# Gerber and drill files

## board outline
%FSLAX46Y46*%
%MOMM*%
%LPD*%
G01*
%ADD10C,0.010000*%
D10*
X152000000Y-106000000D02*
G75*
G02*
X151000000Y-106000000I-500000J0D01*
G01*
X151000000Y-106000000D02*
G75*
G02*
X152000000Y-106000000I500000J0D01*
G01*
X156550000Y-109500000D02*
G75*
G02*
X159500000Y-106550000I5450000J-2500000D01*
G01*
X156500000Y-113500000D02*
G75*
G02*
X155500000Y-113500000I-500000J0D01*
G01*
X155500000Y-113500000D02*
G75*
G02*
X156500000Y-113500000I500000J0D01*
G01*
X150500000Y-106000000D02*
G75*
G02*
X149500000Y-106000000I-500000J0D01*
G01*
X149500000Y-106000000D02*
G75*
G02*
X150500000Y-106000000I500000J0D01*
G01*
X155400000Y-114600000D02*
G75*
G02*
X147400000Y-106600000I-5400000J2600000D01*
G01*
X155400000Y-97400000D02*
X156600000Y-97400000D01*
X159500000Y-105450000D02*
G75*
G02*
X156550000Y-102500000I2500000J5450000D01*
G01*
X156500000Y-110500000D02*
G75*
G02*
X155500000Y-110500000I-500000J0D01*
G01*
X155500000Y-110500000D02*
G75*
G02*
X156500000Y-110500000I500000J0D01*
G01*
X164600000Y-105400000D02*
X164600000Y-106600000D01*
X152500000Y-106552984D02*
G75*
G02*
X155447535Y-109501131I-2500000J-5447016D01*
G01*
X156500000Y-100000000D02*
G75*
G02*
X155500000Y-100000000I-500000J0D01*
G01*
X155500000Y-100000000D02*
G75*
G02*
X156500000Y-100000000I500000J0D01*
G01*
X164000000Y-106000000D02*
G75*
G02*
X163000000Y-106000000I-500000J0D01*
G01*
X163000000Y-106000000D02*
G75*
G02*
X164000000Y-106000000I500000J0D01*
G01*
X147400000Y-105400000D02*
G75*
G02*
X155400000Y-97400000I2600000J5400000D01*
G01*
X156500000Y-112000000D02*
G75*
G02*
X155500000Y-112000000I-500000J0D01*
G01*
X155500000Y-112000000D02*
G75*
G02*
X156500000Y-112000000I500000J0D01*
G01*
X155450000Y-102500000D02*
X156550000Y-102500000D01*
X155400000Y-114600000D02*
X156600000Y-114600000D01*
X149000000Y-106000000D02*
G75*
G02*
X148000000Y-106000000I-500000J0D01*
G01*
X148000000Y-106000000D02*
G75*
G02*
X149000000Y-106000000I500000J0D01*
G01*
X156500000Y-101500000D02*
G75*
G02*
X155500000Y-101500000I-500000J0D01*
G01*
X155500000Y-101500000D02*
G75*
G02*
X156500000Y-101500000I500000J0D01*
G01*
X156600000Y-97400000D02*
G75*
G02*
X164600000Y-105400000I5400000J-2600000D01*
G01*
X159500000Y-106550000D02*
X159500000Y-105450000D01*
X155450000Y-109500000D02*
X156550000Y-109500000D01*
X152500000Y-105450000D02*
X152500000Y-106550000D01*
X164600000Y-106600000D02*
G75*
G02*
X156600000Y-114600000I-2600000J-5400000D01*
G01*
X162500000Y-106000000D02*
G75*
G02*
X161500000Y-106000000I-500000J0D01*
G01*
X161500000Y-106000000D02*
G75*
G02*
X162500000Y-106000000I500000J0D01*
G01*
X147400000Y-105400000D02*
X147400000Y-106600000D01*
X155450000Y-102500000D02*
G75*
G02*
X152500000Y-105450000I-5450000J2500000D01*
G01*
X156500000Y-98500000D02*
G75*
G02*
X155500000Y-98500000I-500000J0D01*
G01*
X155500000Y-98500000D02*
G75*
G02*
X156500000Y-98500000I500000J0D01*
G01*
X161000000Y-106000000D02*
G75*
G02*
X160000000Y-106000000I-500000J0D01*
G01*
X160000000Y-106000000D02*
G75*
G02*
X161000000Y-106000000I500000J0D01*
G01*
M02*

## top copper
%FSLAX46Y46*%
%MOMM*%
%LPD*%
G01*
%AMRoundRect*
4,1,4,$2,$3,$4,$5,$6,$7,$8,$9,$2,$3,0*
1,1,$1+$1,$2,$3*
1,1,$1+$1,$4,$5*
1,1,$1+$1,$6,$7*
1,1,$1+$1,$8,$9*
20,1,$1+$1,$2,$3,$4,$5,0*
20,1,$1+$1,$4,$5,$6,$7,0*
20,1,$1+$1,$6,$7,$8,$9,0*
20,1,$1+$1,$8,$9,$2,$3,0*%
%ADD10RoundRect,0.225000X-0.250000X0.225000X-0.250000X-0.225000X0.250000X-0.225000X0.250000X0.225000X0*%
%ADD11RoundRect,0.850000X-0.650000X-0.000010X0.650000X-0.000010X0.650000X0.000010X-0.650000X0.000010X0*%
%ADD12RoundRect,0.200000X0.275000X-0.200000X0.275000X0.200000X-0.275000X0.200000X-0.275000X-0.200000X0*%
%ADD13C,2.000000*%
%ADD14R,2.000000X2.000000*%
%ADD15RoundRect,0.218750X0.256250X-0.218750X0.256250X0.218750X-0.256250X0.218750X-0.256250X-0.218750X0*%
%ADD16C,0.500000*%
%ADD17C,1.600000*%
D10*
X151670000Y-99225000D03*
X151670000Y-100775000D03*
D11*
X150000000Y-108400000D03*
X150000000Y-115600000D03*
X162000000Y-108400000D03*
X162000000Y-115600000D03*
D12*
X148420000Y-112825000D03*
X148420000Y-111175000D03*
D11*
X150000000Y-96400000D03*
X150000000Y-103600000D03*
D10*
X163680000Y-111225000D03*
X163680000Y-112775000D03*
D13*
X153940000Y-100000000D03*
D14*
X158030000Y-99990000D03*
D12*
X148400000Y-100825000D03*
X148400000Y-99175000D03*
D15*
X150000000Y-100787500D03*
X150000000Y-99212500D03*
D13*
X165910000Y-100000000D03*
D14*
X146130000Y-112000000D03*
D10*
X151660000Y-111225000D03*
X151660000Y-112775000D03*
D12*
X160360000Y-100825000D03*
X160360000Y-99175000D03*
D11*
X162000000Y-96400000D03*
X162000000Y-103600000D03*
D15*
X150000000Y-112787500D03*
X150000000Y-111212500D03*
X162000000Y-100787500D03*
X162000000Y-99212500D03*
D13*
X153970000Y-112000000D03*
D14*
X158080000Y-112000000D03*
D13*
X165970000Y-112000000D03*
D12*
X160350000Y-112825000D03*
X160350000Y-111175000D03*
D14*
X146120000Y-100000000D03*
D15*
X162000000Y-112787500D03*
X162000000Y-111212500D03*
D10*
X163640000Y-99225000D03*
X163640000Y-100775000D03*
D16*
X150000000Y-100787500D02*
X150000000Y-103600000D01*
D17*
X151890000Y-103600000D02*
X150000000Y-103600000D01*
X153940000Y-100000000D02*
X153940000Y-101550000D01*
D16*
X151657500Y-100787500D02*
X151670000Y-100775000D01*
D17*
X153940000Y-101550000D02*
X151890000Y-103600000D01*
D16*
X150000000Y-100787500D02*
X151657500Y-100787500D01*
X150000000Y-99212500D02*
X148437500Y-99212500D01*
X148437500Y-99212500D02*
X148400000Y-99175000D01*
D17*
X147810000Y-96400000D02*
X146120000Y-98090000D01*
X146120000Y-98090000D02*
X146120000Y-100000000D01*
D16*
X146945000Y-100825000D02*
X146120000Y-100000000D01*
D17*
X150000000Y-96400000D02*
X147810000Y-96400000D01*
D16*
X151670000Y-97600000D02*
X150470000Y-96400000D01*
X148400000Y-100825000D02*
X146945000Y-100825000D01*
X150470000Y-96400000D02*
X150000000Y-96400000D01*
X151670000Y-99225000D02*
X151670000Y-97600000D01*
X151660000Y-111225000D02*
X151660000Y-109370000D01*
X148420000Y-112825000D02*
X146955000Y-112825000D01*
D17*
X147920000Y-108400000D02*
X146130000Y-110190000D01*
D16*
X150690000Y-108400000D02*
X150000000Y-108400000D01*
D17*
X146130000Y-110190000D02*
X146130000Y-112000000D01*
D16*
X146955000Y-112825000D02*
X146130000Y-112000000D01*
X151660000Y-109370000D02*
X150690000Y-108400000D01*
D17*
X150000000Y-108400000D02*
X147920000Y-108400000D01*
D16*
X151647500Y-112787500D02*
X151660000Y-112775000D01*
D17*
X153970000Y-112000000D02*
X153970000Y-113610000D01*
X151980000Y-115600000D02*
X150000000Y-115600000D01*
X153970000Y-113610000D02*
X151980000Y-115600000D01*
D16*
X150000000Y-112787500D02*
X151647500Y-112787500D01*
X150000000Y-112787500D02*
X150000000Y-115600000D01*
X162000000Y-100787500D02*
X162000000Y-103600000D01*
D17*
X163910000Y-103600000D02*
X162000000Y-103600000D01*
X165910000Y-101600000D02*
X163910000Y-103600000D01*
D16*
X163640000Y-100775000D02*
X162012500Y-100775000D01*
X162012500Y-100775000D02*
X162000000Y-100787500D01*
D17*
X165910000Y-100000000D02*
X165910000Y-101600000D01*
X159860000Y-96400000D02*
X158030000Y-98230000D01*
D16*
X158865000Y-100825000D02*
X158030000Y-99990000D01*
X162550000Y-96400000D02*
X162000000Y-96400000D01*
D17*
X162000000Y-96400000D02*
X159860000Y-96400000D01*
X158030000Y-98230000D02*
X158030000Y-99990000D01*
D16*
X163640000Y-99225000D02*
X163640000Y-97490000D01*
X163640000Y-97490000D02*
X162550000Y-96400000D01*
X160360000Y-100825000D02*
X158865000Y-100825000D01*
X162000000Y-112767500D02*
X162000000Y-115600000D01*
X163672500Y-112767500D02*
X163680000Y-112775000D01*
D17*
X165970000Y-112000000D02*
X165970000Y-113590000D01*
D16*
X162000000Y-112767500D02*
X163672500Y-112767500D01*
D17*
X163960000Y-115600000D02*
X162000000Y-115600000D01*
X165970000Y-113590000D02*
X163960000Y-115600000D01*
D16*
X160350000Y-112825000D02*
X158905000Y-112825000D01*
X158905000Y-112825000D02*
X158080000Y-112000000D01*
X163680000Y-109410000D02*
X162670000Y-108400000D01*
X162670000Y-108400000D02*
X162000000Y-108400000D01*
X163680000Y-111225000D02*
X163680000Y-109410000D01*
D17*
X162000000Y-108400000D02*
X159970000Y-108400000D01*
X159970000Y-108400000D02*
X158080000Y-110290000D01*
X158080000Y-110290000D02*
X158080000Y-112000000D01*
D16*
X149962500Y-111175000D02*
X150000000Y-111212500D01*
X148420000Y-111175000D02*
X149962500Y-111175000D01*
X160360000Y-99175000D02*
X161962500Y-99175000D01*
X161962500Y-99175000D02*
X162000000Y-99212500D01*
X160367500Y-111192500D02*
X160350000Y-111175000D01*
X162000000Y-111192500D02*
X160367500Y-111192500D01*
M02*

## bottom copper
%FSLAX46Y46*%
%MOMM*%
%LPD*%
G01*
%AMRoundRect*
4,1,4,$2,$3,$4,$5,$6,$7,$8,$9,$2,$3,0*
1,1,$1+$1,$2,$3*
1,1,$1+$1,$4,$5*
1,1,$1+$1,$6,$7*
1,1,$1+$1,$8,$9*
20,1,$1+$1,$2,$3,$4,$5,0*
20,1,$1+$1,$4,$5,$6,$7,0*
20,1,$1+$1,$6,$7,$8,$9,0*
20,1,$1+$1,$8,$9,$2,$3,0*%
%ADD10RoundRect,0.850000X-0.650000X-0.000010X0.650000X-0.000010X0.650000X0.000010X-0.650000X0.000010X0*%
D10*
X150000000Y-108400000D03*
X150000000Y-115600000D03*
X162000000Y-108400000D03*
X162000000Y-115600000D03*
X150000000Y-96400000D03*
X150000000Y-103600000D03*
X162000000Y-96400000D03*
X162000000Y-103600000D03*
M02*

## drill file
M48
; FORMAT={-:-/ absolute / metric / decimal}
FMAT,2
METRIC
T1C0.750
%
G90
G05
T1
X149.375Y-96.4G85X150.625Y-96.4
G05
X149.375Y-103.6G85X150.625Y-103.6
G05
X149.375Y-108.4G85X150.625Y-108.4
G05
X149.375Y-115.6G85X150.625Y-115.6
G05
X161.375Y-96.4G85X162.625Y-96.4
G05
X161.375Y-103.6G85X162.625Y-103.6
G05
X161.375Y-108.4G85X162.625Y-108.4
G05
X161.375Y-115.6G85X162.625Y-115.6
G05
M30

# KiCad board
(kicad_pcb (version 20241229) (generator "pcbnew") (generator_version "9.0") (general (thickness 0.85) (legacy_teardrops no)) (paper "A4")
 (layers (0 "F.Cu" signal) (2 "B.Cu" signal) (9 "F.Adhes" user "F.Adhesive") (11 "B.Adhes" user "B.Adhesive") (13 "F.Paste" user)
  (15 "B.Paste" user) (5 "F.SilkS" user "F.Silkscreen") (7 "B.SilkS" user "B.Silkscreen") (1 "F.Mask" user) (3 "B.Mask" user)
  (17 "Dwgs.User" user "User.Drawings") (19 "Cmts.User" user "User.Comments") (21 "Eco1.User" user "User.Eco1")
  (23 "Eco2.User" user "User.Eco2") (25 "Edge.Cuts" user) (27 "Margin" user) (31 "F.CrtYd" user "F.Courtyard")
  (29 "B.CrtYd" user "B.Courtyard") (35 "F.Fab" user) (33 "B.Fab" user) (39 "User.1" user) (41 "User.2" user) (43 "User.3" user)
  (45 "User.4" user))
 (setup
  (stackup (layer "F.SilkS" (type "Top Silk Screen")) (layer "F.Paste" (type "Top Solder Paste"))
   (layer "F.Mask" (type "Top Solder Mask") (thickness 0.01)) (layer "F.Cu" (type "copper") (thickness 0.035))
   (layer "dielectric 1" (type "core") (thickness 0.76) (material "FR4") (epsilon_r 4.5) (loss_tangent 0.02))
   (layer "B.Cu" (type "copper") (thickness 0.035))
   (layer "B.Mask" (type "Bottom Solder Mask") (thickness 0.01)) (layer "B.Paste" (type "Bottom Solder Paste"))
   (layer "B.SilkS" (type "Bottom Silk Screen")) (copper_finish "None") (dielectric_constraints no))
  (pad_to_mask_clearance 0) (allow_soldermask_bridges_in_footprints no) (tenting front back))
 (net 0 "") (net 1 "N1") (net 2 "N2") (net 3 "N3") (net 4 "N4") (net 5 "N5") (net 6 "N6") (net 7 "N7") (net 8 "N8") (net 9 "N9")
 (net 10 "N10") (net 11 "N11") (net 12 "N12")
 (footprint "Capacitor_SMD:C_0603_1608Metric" (layer "F.Cu") (at 151.67 100 -90)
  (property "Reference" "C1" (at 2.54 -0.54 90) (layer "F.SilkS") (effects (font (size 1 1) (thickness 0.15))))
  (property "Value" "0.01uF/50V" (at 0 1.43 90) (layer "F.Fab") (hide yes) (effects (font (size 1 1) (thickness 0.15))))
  (pad "1" smd roundrect (at -0.775 0 270) (size 0.9 0.95) (layers "F.Cu" "F.Mask" "F.Paste") (roundrect_rratio 0.25) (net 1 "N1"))
  (pad "2" smd roundrect (at 0.775 0 270) (size 0.9 0.95) (layers "F.Cu" "F.Mask" "F.Paste") (roundrect_rratio 0.25) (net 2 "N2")))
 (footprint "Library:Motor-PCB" (layer "F.Cu") (at 150 112)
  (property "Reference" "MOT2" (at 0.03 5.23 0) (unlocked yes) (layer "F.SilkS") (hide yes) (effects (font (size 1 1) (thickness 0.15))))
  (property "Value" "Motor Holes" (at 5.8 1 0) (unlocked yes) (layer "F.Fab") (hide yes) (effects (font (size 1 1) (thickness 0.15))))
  (pad "1" thru_hole roundrect (at 0 -3.6) (size 3 1.7) (drill oval 2 0.75) (layers "*.Cu" "*.Mask") (remove_unused_layers no)
   (roundrect_rratio 0.5) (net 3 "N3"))
  (pad "2" thru_hole roundrect (at 0 3.6) (size 3 1.7) (drill oval 2 0.75) (layers "*.Cu" "*.Mask") (remove_unused_layers no)
   (roundrect_rratio 0.5) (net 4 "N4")))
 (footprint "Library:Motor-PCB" (layer "F.Cu") (at 162 112)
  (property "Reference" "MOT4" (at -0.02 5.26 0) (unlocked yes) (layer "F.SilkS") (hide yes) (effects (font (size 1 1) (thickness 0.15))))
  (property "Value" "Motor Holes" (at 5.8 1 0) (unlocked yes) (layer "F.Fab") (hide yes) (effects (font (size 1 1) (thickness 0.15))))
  (pad "1" thru_hole roundrect (at 0 -3.6) (size 3 1.7) (drill oval 2 0.75) (layers "*.Cu" "*.Mask") (remove_unused_layers no)
   (roundrect_rratio 0.5) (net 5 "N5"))
  (pad "2" thru_hole roundrect (at 0 3.6) (size 3 1.7) (drill oval 2 0.75) (layers "*.Cu" "*.Mask") (remove_unused_layers no)
   (roundrect_rratio 0.5) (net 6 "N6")))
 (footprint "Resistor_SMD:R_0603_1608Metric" (layer "F.Cu") (at 148.42 112 90)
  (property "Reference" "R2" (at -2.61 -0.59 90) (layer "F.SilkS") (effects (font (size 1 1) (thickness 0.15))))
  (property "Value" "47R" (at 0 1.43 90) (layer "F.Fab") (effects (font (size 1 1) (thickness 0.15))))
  (pad "1" smd roundrect (at -0.825 0 90) (size 0.8 0.95) (layers "F.Cu" "F.Mask" "F.Paste") (roundrect_rratio 0.25) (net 3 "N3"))
  (pad "2" smd roundrect (at 0.825 0 90) (size 0.8 0.95) (layers "F.Cu" "F.Mask" "F.Paste") (roundrect_rratio 0.25) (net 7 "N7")))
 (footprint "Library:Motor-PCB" (layer "F.Cu") (at 150 100)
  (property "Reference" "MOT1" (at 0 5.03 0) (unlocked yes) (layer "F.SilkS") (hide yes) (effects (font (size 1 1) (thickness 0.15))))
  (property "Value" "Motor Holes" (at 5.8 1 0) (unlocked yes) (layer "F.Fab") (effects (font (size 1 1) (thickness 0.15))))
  (pad "1" thru_hole roundrect (at 0 -3.6) (size 3 1.7) (drill oval 2 0.75) (layers "*.Cu" "*.Mask") (remove_unused_layers no)
   (roundrect_rratio 0.5) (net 1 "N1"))
  (pad "2" thru_hole roundrect (at 0 3.6) (size 3 1.7) (drill oval 2 0.75) (layers "*.Cu" "*.Mask") (remove_unused_layers no)
   (roundrect_rratio 0.5) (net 2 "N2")))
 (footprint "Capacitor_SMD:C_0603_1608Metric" (layer "F.Cu") (at 163.68 112 -90)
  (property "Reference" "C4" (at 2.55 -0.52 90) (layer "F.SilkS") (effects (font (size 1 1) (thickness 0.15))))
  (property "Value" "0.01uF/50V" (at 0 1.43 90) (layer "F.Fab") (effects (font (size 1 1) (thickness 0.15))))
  (pad "1" smd roundrect (at -0.775 0 270) (size 0.9 0.95) (layers "F.Cu" "F.Mask" "F.Paste") (roundrect_rratio 0.25) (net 5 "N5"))
  (pad "2" smd roundrect (at 0.775 0 270) (size 0.9 0.95) (layers "F.Cu" "F.Mask" "F.Paste") (roundrect_rratio 0.25) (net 6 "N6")))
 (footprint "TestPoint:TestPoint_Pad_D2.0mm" (layer "F.Cu") (at 153.94 100)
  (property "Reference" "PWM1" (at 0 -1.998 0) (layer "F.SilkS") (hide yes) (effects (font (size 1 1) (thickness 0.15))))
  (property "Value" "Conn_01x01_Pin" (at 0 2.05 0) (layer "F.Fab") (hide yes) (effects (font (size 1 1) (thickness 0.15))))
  (pad "1" smd circle (at 0 0) (size 2 2) (layers "F.Cu" "F.Mask") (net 2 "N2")))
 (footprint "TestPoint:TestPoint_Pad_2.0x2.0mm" (layer "F.Cu") (at 158.03 99.99)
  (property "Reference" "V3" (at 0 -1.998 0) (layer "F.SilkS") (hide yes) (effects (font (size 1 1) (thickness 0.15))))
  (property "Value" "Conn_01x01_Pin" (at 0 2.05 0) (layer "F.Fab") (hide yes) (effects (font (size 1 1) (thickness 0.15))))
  (pad "1" smd rect (at 0 0) (size 2 2) (layers "F.Cu" "F.Mask") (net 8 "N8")))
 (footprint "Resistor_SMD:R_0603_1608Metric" (layer "F.Cu") (at 148.4 100 90)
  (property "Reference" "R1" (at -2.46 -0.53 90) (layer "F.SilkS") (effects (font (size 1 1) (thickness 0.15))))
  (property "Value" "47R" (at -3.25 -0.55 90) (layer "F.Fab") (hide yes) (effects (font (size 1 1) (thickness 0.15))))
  (pad "1" smd roundrect (at -0.825 0 90) (size 0.8 0.95) (layers "F.Cu" "F.Mask" "F.Paste") (roundrect_rratio 0.25) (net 1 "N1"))
  (pad "2" smd roundrect (at 0.825 0 90) (size 0.8 0.95) (layers "F.Cu" "F.Mask" "F.Paste") (roundrect_rratio 0.25) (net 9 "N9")))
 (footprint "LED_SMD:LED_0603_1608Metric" (layer "F.Cu") (at 150 100 90)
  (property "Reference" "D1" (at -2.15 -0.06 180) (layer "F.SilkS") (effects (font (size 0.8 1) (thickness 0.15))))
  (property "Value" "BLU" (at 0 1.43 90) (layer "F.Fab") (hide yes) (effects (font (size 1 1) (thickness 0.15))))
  (pad "1" smd roundrect (at -0.7875 0 90) (size 0.875 0.95) (layers "F.Cu" "F.Mask" "F.Paste") (roundrect_rratio 0.25) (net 2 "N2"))
  (pad "2" smd roundrect (at 0.7875 0 90) (size 0.875 0.95) (layers "F.Cu" "F.Mask" "F.Paste") (roundrect_rratio 0.25) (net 9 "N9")))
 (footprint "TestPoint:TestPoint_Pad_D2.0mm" (layer "F.Cu") (at 165.91 100 90)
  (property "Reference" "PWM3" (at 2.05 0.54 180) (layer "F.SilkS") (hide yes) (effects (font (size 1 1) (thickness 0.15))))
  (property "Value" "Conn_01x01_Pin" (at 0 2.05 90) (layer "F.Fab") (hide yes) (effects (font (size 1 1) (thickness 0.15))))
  (pad "1" smd circle (at 0 0 90) (size 2 2) (layers "F.Cu" "F.Mask") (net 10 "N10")))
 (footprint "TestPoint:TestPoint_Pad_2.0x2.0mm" (layer "F.Cu") (at 146.13 112)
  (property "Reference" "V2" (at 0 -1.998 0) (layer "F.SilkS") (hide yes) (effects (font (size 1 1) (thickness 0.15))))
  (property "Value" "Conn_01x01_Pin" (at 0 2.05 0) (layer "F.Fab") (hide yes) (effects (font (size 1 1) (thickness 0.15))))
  (pad "1" smd rect (at 0 0) (size 2 2) (layers "F.Cu" "F.Mask") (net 3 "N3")))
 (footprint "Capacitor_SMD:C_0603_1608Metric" (layer "F.Cu") (at 151.66 112 -90)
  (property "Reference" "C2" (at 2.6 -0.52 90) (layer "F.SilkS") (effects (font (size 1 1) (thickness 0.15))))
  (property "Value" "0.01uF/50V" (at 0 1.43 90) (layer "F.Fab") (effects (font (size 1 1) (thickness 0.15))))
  (pad "1" smd roundrect (at -0.775 0 270) (size 0.9 0.95) (layers "F.Cu" "F.Mask" "F.Paste") (roundrect_rratio 0.25) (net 3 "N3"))
  (pad "2" smd roundrect (at 0.775 0 270) (size 0.9 0.95) (layers "F.Cu" "F.Mask" "F.Paste") (roundrect_rratio 0.25) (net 4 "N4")))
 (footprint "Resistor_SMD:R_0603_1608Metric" (layer "F.Cu") (at 160.36 100 90)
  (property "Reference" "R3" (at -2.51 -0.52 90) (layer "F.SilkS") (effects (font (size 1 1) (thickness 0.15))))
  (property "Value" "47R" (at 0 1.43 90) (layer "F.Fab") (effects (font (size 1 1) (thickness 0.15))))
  (pad "1" smd roundrect (at -0.825 0 90) (size 0.8 0.95) (layers "F.Cu" "F.Mask" "F.Paste") (roundrect_rratio 0.25) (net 8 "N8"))
  (pad "2" smd roundrect (at 0.825 0 90) (size 0.8 0.95) (layers "F.Cu" "F.Mask" "F.Paste") (roundrect_rratio 0.25) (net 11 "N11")))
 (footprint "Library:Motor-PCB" (layer "F.Cu") (at 162 100)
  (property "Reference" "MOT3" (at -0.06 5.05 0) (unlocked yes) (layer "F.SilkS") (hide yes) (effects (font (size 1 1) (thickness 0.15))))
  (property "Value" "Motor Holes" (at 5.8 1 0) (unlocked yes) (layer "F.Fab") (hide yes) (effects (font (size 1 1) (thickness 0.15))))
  (pad "1" thru_hole roundrect (at 0 -3.6) (size 3 1.7) (drill oval 2 0.75) (layers "*.Cu" "*.Mask") (remove_unused_layers no)
   (roundrect_rratio 0.5) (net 8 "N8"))
  (pad "2" thru_hole roundrect (at 0 3.6) (size 3 1.7) (drill oval 2 0.75) (layers "*.Cu" "*.Mask") (remove_unused_layers no)
   (roundrect_rratio 0.5) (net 10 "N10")))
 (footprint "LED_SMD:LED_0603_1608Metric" (layer "F.Cu") (at 150 112 90)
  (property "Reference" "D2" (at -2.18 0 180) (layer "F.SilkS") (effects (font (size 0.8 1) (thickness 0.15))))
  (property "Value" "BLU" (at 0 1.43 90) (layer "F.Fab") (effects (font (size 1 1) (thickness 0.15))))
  (pad "1" smd roundrect (at -0.7875 0 90) (size 0.875 0.95) (layers "F.Cu" "F.Mask" "F.Paste") (roundrect_rratio 0.25) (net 4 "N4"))
  (pad "2" smd roundrect (at 0.7875 0 90) (size 0.875 0.95) (layers "F.Cu" "F.Mask" "F.Paste") (roundrect_rratio 0.25) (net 7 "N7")))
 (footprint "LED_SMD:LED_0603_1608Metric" (layer "F.Cu") (at 162 100 90)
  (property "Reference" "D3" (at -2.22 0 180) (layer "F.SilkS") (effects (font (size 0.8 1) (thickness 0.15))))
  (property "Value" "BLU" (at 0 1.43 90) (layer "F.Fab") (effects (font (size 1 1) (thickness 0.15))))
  (pad "1" smd roundrect (at -0.7875 0 90) (size 0.875 0.95) (layers "F.Cu" "F.Mask" "F.Paste") (roundrect_rratio 0.25) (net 10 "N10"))
  (pad "2" smd roundrect (at 0.7875 0 90) (size 0.875 0.95) (layers "F.Cu" "F.Mask" "F.Paste") (roundrect_rratio 0.25) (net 11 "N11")))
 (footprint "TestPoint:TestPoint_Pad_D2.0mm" (layer "F.Cu") (at 153.97 112)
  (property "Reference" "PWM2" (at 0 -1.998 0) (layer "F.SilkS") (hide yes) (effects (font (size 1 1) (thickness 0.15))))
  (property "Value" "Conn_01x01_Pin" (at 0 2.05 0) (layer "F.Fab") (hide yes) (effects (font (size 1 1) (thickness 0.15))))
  (pad "1" smd circle (at 0 0) (size 2 2) (layers "F.Cu" "F.Mask") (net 4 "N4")))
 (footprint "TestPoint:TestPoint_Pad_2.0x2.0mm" (layer "F.Cu") (at 158.08 112)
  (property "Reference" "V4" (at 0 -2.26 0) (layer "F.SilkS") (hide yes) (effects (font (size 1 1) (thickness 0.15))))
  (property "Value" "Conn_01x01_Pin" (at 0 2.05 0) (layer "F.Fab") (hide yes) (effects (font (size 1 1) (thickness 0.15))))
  (pad "1" smd rect (at 0 0) (size 2 2) (layers "F.Cu" "F.Mask") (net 5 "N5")))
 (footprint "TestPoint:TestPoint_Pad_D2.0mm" (layer "F.Cu") (at 165.97 112)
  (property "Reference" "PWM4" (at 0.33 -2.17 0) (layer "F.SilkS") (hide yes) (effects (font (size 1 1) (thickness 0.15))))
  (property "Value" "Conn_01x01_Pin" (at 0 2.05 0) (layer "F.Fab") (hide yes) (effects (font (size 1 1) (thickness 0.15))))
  (pad "1" smd circle (at 0 0) (size 2 2) (layers "F.Cu" "F.Mask") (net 6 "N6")))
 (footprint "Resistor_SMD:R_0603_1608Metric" (layer "F.Cu") (at 160.35 112 90)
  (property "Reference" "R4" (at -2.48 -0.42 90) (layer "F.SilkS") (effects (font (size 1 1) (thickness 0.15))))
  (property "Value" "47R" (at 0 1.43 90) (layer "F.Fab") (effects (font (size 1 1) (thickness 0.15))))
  (pad "1" smd roundrect (at -0.825 0 90) (size 0.8 0.95) (layers "F.Cu" "F.Mask" "F.Paste") (roundrect_rratio 0.25) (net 5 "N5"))
  (pad "2" smd roundrect (at 0.825 0 90) (size 0.8 0.95) (layers "F.Cu" "F.Mask" "F.Paste") (roundrect_rratio 0.25) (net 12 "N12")))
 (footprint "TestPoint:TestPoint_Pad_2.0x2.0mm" (layer "F.Cu") (at 146.12 100)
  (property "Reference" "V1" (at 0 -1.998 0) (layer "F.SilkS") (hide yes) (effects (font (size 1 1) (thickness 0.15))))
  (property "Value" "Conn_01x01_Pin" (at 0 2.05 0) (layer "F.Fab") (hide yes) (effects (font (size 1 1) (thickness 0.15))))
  (pad "1" smd rect (at 0 0) (size 2 2) (layers "F.Cu" "F.Mask") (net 1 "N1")))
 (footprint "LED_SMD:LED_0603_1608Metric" (layer "F.Cu") (at 162 112 90)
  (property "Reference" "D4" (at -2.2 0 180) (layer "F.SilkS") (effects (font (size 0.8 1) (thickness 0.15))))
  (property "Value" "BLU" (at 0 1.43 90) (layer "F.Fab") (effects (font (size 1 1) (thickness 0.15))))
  (pad "1" smd roundrect (at -0.7875 0 90) (size 0.875 0.95) (layers "F.Cu" "F.Mask" "F.Paste") (roundrect_rratio 0.25) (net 6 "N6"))
  (pad "2" smd roundrect (at 0.7875 0 90) (size 0.875 0.95) (layers "F.Cu" "F.Mask" "F.Paste") (roundrect_rratio 0.25) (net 12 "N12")))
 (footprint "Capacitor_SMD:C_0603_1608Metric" (layer "F.Cu") (at 163.64 100 -90)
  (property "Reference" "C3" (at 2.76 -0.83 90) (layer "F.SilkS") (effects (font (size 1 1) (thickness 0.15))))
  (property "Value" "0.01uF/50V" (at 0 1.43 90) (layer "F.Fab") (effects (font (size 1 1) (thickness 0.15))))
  (pad "1" smd roundrect (at -0.775 0 270) (size 0.9 0.95) (layers "F.Cu" "F.Mask" "F.Paste") (roundrect_rratio 0.25) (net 8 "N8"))
  (pad "2" smd roundrect (at 0.775 0 270) (size 0.9 0.95) (layers "F.Cu" "F.Mask" "F.Paste") (roundrect_rratio 0.25) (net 10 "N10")))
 (gr_circle (center 151.5 106) (end 151.5 105.5) (stroke (width 0.01) (type solid)) (fill no) (layer "Edge.Cuts"))
 (gr_arc (start 156.55 109.5) (mid 157.760159 107.760159) (end 159.5 106.55) (stroke (width 0.01) (type solid)) (layer "Edge.Cuts"))
 (gr_circle (center 156 113.5) (end 155.5 113.5) (stroke (width 0.01) (type solid)) (fill no) (layer "Edge.Cuts"))
 (gr_circle (center 150 106) (end 150 105.5) (stroke (width 0.01) (type solid)) (fill no) (layer "Edge.Cuts"))
 (gr_arc (start 155.4 114.6) (mid 145.762076 116.237924) (end 147.4 106.6) (stroke (width 0.01) (type solid)) (layer "Edge.Cuts"))
 (gr_line (start 155.4 97.4) (end 156.6 97.4) (stroke (width 0.01) (type solid)) (layer "Edge.Cuts"))
 (gr_arc (start 159.5 105.45) (mid 157.760159 104.239841) (end 156.55 102.5) (stroke (width 0.01) (type solid)) (layer "Edge.Cuts"))
 (gr_circle (center 156 110.5) (end 155.5 110.5) (stroke (width 0.01) (type solid)) (fill no) (layer "Edge.Cuts"))
 (gr_line (start 164.6 105.4) (end 164.6 106.6) (stroke (width 0.01) (type solid)) (layer "Edge.Cuts"))
 (gr_arc (start 152.5 106.552984) (mid 154.238363 107.762517) (end 155.447535 109.501131) (stroke (width 0.01) (type solid))
  (layer "Edge.Cuts"))
 (gr_circle (center 156 100) (end 155.5 100) (stroke (width 0.01) (type solid)) (fill no) (layer "Edge.Cuts"))
 (gr_circle (center 163.5 106) (end 163.5 105.5) (stroke (width 0.01) (type solid)) (fill no) (layer "Edge.Cuts"))
 (gr_arc (start 147.4 105.4) (mid 145.762076 95.762076) (end 155.4 97.4) (stroke (width 0.01) (type solid)) (layer "Edge.Cuts"))
 (gr_circle (center 156 112) (end 155.5 112) (stroke (width 0.01) (type solid)) (fill no) (layer "Edge.Cuts"))
 (gr_line (start 155.45 102.5) (end 156.55 102.5) (stroke (width 0.01) (type solid)) (layer "Edge.Cuts"))
 (gr_line (start 155.4 114.6) (end 156.6 114.6) (stroke (width 0.01) (type solid)) (layer "Edge.Cuts"))
 (gr_circle (center 148.5 106) (end 148.5 105.5) (stroke (width 0.01) (type solid)) (fill no) (layer "Edge.Cuts"))
 (gr_circle (center 156 101.5) (end 155.5 101.5) (stroke (width 0.01) (type solid)) (fill no) (layer "Edge.Cuts"))
 (gr_arc (start 156.6 97.4) (mid 166.237924 95.762076) (end 164.6 105.4) (stroke (width 0.01) (type solid)) (layer "Edge.Cuts"))
 (gr_line (start 159.5 106.55) (end 159.5 105.45) (stroke (width 0.01) (type solid)) (layer "Edge.Cuts"))
 (gr_line (start 155.45 109.5) (end 156.55 109.5) (stroke (width 0.01) (type solid)) (layer "Edge.Cuts"))
 (gr_line (start 152.5 105.45) (end 152.5 106.55) (stroke (width 0.01) (type solid)) (layer "Edge.Cuts"))
 (gr_arc (start 164.6 106.6) (mid 166.237924 116.237924) (end 156.6 114.6) (stroke (width 0.01) (type solid)) (layer "Edge.Cuts"))
 (gr_circle (center 162 106) (end 162 105.5) (stroke (width 0.01) (type solid)) (fill no) (layer "Edge.Cuts"))
 (gr_line (start 147.4 105.4) (end 147.4 106.6) (stroke (width 0.01) (type solid)) (layer "Edge.Cuts"))
 (gr_arc (start 155.45 102.5) (mid 154.239841 104.239841) (end 152.5 105.45) (stroke (width 0.01) (type solid)) (layer "Edge.Cuts"))
 (gr_circle (center 156 98.5) (end 155.5 98.5) (stroke (width 0.01) (type solid)) (fill no) (layer "Edge.Cuts"))
 (gr_circle (center 160.5 106) (end 160.5 105.5) (stroke (width 0.01) (type solid)) (fill no) (layer "Edge.Cuts"))
 (segment (start 150 100.7875) (end 150 103.6) (width 0.5) (layer "F.Cu") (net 2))
 (segment (start 151.89 103.6) (end 150 103.6) (width 1.6) (layer "F.Cu") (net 2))
 (segment (start 153.94 100) (end 153.94 101.55) (width 1.6) (layer "F.Cu") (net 2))
 (segment (start 151.6575 100.7875) (end 151.67 100.775) (width 0.5) (layer "F.Cu") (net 2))
 (segment (start 153.94 101.55) (end 151.89 103.6) (width 1.6) (layer "F.Cu") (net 2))
 (segment (start 150 100.7875) (end 151.6575 100.7875) (width 0.5) (layer "F.Cu") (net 2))
 (segment (start 150 99.2125) (end 148.4375 99.2125) (width 0.5) (layer "F.Cu") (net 9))
 (segment (start 148.4375 99.2125) (end 148.4 99.175) (width 0.5) (layer "F.Cu") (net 9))
 (segment (start 147.81 96.4) (end 146.12 98.09) (width 1.6) (layer "F.Cu") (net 1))
 (segment (start 146.12 98.09) (end 146.12 100) (width 1.6) (layer "F.Cu") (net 1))
 (segment (start 146.945 100.825) (end 146.12 100) (width 0.5) (layer "F.Cu") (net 1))
 (segment (start 150 96.4) (end 147.81 96.4) (width 1.6) (layer "F.Cu") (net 1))
 (segment (start 151.67 97.6) (end 150.47 96.4) (width 0.5) (layer "F.Cu") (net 1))
 (segment (start 148.4 100.825) (end 146.945 100.825) (width 0.5) (layer "F.Cu") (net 1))
 (segment (start 150.47 96.4) (end 150 96.4) (width 0.5) (layer "F.Cu") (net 1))
 (segment (start 151.67 99.225) (end 151.67 97.6) (width 0.5) (layer "F.Cu") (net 1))
 (segment (start 151.66 111.225) (end 151.66 109.37) (width 0.5) (layer "F.Cu") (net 3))
 (segment (start 148.42 112.825) (end 146.955 112.825) (width 0.5) (layer "F.Cu") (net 3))
 (segment (start 147.92 108.4) (end 146.13 110.19) (width 1.6) (layer "F.Cu") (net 3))
 (segment (start 150.69 108.4) (end 150 108.4) (width 0.5) (layer "F.Cu") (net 3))
 (segment (start 146.13 110.19) (end 146.13 112) (width 1.6) (layer "F.Cu") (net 3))
 (segment (start 146.955 112.825) (end 146.13 112) (width 0.5) (layer "F.Cu") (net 3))
 (segment (start 151.66 109.37) (end 150.69 108.4) (width 0.5) (layer "F.Cu") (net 3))
 (segment (start 150 108.4) (end 147.92 108.4) (width 1.6) (layer "F.Cu") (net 3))
 (segment (start 151.6475 112.7875) (end 151.66 112.775) (width 0.5) (layer "F.Cu") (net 4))
 (segment (start 153.97 112) (end 153.97 113.61) (width 1.6) (layer "F.Cu") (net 4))
 (segment (start 151.98 115.6) (end 150 115.6) (width 1.6) (layer "F.Cu") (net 4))
 (segment (start 153.97 113.61) (end 151.98 115.6) (width 1.6) (layer "F.Cu") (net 4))
 (segment (start 150 112.7875) (end 151.6475 112.7875) (width 0.5) (layer "F.Cu") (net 4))
 (segment (start 150 112.7875) (end 150 115.6) (width 0.5) (layer "F.Cu") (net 4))
 (segment (start 162 100.7875) (end 162 103.6) (width 0.5) (layer "F.Cu") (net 10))
 (segment (start 163.91 103.6) (end 162 103.6) (width 1.6) (layer "F.Cu") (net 10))
 (segment (start 165.91 101.6) (end 163.91 103.6) (width 1.6) (layer "F.Cu") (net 10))
 (segment (start 163.64 100.775) (end 162.0125 100.775) (width 0.5) (layer "F.Cu") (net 10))
 (segment (start 162.0125 100.775) (end 162 100.7875) (width 0.5) (layer "F.Cu") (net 10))
 (segment (start 165.91 100) (end 165.91 101.6) (width 1.6) (layer "F.Cu") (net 10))
 (segment (start 159.86 96.4) (end 158.03 98.23) (width 1.6) (layer "F.Cu") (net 8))
 (segment (start 158.865 100.825) (end 158.03 99.99) (width 0.5) (layer "F.Cu") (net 8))
 (segment (start 162.55 96.4) (end 162 96.4) (width 0.5) (layer "F.Cu") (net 8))
 (segment (start 162 96.4) (end 159.86 96.4) (width 1.6) (layer "F.Cu") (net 8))
 (segment (start 158.03 98.23) (end 158.03 99.99) (width 1.6) (layer "F.Cu") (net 8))
 (segment (start 163.64 99.225) (end 163.64 97.49) (width 0.5) (layer "F.Cu") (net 8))
 (segment (start 163.64 97.49) (end 162.55 96.4) (width 0.5) (layer "F.Cu") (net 8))
 (segment (start 160.36 100.825) (end 158.865 100.825) (width 0.5) (layer "F.Cu") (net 8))
 (segment (start 162 112.7675) (end 162 115.6) (width 0.5) (layer "F.Cu") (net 6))
 (segment (start 163.6725 112.7675) (end 163.68 112.775) (width 0.5) (layer "F.Cu") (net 6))
 (segment (start 165.97 112) (end 165.97 113.59) (width 1.6) (layer "F.Cu") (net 6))
 (segment (start 162 112.7675) (end 163.6725 112.7675) (width 0.5) (layer "F.Cu") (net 6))
 (segment (start 163.96 115.6) (end 162 115.6) (width 1.6) (layer "F.Cu") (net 6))
 (segment (start 165.97 113.59) (end 163.96 115.6) (width 1.6) (layer "F.Cu") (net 6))
 (segment (start 160.35 112.825) (end 158.905 112.825) (width 0.5) (layer "F.Cu") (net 5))
 (segment (start 158.905 112.825) (end 158.08 112) (width 0.5) (layer "F.Cu") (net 5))
 (segment (start 163.68 109.41) (end 162.67 108.4) (width 0.5) (layer "F.Cu") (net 5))
 (segment (start 162.67 108.4) (end 162 108.4) (width 0.5) (layer "F.Cu") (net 5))
 (segment (start 163.68 111.225) (end 163.68 109.41) (width 0.5) (layer "F.Cu") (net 5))
 (segment (start 162 108.4) (end 159.97 108.4) (width 1.6) (layer "F.Cu") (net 5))
 (segment (start 159.97 108.4) (end 158.08 110.29) (width 1.6) (layer "F.Cu") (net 5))
 (segment (start 158.08 110.29) (end 158.08 112) (width 1.6) (layer "F.Cu") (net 5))
 (segment (start 149.9625 111.175) (end 150 111.2125) (width 0.5) (layer "F.Cu") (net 7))
 (segment (start 148.42 111.175) (end 149.9625 111.175) (width 0.5) (layer "F.Cu") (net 7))
 (segment (start 160.36 99.175) (end 161.9625 99.175) (width 0.5) (layer "F.Cu") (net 11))
 (segment (start 161.9625 99.175) (end 162 99.2125) (width 0.5) (layer "F.Cu") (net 11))
 (segment (start 160.3675 111.1925) (end 160.35 111.175) (width 0.5) (layer "F.Cu") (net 12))
 (segment (start 162 111.1925) (end 160.3675 111.1925) (width 0.5) (layer "F.Cu") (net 12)))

